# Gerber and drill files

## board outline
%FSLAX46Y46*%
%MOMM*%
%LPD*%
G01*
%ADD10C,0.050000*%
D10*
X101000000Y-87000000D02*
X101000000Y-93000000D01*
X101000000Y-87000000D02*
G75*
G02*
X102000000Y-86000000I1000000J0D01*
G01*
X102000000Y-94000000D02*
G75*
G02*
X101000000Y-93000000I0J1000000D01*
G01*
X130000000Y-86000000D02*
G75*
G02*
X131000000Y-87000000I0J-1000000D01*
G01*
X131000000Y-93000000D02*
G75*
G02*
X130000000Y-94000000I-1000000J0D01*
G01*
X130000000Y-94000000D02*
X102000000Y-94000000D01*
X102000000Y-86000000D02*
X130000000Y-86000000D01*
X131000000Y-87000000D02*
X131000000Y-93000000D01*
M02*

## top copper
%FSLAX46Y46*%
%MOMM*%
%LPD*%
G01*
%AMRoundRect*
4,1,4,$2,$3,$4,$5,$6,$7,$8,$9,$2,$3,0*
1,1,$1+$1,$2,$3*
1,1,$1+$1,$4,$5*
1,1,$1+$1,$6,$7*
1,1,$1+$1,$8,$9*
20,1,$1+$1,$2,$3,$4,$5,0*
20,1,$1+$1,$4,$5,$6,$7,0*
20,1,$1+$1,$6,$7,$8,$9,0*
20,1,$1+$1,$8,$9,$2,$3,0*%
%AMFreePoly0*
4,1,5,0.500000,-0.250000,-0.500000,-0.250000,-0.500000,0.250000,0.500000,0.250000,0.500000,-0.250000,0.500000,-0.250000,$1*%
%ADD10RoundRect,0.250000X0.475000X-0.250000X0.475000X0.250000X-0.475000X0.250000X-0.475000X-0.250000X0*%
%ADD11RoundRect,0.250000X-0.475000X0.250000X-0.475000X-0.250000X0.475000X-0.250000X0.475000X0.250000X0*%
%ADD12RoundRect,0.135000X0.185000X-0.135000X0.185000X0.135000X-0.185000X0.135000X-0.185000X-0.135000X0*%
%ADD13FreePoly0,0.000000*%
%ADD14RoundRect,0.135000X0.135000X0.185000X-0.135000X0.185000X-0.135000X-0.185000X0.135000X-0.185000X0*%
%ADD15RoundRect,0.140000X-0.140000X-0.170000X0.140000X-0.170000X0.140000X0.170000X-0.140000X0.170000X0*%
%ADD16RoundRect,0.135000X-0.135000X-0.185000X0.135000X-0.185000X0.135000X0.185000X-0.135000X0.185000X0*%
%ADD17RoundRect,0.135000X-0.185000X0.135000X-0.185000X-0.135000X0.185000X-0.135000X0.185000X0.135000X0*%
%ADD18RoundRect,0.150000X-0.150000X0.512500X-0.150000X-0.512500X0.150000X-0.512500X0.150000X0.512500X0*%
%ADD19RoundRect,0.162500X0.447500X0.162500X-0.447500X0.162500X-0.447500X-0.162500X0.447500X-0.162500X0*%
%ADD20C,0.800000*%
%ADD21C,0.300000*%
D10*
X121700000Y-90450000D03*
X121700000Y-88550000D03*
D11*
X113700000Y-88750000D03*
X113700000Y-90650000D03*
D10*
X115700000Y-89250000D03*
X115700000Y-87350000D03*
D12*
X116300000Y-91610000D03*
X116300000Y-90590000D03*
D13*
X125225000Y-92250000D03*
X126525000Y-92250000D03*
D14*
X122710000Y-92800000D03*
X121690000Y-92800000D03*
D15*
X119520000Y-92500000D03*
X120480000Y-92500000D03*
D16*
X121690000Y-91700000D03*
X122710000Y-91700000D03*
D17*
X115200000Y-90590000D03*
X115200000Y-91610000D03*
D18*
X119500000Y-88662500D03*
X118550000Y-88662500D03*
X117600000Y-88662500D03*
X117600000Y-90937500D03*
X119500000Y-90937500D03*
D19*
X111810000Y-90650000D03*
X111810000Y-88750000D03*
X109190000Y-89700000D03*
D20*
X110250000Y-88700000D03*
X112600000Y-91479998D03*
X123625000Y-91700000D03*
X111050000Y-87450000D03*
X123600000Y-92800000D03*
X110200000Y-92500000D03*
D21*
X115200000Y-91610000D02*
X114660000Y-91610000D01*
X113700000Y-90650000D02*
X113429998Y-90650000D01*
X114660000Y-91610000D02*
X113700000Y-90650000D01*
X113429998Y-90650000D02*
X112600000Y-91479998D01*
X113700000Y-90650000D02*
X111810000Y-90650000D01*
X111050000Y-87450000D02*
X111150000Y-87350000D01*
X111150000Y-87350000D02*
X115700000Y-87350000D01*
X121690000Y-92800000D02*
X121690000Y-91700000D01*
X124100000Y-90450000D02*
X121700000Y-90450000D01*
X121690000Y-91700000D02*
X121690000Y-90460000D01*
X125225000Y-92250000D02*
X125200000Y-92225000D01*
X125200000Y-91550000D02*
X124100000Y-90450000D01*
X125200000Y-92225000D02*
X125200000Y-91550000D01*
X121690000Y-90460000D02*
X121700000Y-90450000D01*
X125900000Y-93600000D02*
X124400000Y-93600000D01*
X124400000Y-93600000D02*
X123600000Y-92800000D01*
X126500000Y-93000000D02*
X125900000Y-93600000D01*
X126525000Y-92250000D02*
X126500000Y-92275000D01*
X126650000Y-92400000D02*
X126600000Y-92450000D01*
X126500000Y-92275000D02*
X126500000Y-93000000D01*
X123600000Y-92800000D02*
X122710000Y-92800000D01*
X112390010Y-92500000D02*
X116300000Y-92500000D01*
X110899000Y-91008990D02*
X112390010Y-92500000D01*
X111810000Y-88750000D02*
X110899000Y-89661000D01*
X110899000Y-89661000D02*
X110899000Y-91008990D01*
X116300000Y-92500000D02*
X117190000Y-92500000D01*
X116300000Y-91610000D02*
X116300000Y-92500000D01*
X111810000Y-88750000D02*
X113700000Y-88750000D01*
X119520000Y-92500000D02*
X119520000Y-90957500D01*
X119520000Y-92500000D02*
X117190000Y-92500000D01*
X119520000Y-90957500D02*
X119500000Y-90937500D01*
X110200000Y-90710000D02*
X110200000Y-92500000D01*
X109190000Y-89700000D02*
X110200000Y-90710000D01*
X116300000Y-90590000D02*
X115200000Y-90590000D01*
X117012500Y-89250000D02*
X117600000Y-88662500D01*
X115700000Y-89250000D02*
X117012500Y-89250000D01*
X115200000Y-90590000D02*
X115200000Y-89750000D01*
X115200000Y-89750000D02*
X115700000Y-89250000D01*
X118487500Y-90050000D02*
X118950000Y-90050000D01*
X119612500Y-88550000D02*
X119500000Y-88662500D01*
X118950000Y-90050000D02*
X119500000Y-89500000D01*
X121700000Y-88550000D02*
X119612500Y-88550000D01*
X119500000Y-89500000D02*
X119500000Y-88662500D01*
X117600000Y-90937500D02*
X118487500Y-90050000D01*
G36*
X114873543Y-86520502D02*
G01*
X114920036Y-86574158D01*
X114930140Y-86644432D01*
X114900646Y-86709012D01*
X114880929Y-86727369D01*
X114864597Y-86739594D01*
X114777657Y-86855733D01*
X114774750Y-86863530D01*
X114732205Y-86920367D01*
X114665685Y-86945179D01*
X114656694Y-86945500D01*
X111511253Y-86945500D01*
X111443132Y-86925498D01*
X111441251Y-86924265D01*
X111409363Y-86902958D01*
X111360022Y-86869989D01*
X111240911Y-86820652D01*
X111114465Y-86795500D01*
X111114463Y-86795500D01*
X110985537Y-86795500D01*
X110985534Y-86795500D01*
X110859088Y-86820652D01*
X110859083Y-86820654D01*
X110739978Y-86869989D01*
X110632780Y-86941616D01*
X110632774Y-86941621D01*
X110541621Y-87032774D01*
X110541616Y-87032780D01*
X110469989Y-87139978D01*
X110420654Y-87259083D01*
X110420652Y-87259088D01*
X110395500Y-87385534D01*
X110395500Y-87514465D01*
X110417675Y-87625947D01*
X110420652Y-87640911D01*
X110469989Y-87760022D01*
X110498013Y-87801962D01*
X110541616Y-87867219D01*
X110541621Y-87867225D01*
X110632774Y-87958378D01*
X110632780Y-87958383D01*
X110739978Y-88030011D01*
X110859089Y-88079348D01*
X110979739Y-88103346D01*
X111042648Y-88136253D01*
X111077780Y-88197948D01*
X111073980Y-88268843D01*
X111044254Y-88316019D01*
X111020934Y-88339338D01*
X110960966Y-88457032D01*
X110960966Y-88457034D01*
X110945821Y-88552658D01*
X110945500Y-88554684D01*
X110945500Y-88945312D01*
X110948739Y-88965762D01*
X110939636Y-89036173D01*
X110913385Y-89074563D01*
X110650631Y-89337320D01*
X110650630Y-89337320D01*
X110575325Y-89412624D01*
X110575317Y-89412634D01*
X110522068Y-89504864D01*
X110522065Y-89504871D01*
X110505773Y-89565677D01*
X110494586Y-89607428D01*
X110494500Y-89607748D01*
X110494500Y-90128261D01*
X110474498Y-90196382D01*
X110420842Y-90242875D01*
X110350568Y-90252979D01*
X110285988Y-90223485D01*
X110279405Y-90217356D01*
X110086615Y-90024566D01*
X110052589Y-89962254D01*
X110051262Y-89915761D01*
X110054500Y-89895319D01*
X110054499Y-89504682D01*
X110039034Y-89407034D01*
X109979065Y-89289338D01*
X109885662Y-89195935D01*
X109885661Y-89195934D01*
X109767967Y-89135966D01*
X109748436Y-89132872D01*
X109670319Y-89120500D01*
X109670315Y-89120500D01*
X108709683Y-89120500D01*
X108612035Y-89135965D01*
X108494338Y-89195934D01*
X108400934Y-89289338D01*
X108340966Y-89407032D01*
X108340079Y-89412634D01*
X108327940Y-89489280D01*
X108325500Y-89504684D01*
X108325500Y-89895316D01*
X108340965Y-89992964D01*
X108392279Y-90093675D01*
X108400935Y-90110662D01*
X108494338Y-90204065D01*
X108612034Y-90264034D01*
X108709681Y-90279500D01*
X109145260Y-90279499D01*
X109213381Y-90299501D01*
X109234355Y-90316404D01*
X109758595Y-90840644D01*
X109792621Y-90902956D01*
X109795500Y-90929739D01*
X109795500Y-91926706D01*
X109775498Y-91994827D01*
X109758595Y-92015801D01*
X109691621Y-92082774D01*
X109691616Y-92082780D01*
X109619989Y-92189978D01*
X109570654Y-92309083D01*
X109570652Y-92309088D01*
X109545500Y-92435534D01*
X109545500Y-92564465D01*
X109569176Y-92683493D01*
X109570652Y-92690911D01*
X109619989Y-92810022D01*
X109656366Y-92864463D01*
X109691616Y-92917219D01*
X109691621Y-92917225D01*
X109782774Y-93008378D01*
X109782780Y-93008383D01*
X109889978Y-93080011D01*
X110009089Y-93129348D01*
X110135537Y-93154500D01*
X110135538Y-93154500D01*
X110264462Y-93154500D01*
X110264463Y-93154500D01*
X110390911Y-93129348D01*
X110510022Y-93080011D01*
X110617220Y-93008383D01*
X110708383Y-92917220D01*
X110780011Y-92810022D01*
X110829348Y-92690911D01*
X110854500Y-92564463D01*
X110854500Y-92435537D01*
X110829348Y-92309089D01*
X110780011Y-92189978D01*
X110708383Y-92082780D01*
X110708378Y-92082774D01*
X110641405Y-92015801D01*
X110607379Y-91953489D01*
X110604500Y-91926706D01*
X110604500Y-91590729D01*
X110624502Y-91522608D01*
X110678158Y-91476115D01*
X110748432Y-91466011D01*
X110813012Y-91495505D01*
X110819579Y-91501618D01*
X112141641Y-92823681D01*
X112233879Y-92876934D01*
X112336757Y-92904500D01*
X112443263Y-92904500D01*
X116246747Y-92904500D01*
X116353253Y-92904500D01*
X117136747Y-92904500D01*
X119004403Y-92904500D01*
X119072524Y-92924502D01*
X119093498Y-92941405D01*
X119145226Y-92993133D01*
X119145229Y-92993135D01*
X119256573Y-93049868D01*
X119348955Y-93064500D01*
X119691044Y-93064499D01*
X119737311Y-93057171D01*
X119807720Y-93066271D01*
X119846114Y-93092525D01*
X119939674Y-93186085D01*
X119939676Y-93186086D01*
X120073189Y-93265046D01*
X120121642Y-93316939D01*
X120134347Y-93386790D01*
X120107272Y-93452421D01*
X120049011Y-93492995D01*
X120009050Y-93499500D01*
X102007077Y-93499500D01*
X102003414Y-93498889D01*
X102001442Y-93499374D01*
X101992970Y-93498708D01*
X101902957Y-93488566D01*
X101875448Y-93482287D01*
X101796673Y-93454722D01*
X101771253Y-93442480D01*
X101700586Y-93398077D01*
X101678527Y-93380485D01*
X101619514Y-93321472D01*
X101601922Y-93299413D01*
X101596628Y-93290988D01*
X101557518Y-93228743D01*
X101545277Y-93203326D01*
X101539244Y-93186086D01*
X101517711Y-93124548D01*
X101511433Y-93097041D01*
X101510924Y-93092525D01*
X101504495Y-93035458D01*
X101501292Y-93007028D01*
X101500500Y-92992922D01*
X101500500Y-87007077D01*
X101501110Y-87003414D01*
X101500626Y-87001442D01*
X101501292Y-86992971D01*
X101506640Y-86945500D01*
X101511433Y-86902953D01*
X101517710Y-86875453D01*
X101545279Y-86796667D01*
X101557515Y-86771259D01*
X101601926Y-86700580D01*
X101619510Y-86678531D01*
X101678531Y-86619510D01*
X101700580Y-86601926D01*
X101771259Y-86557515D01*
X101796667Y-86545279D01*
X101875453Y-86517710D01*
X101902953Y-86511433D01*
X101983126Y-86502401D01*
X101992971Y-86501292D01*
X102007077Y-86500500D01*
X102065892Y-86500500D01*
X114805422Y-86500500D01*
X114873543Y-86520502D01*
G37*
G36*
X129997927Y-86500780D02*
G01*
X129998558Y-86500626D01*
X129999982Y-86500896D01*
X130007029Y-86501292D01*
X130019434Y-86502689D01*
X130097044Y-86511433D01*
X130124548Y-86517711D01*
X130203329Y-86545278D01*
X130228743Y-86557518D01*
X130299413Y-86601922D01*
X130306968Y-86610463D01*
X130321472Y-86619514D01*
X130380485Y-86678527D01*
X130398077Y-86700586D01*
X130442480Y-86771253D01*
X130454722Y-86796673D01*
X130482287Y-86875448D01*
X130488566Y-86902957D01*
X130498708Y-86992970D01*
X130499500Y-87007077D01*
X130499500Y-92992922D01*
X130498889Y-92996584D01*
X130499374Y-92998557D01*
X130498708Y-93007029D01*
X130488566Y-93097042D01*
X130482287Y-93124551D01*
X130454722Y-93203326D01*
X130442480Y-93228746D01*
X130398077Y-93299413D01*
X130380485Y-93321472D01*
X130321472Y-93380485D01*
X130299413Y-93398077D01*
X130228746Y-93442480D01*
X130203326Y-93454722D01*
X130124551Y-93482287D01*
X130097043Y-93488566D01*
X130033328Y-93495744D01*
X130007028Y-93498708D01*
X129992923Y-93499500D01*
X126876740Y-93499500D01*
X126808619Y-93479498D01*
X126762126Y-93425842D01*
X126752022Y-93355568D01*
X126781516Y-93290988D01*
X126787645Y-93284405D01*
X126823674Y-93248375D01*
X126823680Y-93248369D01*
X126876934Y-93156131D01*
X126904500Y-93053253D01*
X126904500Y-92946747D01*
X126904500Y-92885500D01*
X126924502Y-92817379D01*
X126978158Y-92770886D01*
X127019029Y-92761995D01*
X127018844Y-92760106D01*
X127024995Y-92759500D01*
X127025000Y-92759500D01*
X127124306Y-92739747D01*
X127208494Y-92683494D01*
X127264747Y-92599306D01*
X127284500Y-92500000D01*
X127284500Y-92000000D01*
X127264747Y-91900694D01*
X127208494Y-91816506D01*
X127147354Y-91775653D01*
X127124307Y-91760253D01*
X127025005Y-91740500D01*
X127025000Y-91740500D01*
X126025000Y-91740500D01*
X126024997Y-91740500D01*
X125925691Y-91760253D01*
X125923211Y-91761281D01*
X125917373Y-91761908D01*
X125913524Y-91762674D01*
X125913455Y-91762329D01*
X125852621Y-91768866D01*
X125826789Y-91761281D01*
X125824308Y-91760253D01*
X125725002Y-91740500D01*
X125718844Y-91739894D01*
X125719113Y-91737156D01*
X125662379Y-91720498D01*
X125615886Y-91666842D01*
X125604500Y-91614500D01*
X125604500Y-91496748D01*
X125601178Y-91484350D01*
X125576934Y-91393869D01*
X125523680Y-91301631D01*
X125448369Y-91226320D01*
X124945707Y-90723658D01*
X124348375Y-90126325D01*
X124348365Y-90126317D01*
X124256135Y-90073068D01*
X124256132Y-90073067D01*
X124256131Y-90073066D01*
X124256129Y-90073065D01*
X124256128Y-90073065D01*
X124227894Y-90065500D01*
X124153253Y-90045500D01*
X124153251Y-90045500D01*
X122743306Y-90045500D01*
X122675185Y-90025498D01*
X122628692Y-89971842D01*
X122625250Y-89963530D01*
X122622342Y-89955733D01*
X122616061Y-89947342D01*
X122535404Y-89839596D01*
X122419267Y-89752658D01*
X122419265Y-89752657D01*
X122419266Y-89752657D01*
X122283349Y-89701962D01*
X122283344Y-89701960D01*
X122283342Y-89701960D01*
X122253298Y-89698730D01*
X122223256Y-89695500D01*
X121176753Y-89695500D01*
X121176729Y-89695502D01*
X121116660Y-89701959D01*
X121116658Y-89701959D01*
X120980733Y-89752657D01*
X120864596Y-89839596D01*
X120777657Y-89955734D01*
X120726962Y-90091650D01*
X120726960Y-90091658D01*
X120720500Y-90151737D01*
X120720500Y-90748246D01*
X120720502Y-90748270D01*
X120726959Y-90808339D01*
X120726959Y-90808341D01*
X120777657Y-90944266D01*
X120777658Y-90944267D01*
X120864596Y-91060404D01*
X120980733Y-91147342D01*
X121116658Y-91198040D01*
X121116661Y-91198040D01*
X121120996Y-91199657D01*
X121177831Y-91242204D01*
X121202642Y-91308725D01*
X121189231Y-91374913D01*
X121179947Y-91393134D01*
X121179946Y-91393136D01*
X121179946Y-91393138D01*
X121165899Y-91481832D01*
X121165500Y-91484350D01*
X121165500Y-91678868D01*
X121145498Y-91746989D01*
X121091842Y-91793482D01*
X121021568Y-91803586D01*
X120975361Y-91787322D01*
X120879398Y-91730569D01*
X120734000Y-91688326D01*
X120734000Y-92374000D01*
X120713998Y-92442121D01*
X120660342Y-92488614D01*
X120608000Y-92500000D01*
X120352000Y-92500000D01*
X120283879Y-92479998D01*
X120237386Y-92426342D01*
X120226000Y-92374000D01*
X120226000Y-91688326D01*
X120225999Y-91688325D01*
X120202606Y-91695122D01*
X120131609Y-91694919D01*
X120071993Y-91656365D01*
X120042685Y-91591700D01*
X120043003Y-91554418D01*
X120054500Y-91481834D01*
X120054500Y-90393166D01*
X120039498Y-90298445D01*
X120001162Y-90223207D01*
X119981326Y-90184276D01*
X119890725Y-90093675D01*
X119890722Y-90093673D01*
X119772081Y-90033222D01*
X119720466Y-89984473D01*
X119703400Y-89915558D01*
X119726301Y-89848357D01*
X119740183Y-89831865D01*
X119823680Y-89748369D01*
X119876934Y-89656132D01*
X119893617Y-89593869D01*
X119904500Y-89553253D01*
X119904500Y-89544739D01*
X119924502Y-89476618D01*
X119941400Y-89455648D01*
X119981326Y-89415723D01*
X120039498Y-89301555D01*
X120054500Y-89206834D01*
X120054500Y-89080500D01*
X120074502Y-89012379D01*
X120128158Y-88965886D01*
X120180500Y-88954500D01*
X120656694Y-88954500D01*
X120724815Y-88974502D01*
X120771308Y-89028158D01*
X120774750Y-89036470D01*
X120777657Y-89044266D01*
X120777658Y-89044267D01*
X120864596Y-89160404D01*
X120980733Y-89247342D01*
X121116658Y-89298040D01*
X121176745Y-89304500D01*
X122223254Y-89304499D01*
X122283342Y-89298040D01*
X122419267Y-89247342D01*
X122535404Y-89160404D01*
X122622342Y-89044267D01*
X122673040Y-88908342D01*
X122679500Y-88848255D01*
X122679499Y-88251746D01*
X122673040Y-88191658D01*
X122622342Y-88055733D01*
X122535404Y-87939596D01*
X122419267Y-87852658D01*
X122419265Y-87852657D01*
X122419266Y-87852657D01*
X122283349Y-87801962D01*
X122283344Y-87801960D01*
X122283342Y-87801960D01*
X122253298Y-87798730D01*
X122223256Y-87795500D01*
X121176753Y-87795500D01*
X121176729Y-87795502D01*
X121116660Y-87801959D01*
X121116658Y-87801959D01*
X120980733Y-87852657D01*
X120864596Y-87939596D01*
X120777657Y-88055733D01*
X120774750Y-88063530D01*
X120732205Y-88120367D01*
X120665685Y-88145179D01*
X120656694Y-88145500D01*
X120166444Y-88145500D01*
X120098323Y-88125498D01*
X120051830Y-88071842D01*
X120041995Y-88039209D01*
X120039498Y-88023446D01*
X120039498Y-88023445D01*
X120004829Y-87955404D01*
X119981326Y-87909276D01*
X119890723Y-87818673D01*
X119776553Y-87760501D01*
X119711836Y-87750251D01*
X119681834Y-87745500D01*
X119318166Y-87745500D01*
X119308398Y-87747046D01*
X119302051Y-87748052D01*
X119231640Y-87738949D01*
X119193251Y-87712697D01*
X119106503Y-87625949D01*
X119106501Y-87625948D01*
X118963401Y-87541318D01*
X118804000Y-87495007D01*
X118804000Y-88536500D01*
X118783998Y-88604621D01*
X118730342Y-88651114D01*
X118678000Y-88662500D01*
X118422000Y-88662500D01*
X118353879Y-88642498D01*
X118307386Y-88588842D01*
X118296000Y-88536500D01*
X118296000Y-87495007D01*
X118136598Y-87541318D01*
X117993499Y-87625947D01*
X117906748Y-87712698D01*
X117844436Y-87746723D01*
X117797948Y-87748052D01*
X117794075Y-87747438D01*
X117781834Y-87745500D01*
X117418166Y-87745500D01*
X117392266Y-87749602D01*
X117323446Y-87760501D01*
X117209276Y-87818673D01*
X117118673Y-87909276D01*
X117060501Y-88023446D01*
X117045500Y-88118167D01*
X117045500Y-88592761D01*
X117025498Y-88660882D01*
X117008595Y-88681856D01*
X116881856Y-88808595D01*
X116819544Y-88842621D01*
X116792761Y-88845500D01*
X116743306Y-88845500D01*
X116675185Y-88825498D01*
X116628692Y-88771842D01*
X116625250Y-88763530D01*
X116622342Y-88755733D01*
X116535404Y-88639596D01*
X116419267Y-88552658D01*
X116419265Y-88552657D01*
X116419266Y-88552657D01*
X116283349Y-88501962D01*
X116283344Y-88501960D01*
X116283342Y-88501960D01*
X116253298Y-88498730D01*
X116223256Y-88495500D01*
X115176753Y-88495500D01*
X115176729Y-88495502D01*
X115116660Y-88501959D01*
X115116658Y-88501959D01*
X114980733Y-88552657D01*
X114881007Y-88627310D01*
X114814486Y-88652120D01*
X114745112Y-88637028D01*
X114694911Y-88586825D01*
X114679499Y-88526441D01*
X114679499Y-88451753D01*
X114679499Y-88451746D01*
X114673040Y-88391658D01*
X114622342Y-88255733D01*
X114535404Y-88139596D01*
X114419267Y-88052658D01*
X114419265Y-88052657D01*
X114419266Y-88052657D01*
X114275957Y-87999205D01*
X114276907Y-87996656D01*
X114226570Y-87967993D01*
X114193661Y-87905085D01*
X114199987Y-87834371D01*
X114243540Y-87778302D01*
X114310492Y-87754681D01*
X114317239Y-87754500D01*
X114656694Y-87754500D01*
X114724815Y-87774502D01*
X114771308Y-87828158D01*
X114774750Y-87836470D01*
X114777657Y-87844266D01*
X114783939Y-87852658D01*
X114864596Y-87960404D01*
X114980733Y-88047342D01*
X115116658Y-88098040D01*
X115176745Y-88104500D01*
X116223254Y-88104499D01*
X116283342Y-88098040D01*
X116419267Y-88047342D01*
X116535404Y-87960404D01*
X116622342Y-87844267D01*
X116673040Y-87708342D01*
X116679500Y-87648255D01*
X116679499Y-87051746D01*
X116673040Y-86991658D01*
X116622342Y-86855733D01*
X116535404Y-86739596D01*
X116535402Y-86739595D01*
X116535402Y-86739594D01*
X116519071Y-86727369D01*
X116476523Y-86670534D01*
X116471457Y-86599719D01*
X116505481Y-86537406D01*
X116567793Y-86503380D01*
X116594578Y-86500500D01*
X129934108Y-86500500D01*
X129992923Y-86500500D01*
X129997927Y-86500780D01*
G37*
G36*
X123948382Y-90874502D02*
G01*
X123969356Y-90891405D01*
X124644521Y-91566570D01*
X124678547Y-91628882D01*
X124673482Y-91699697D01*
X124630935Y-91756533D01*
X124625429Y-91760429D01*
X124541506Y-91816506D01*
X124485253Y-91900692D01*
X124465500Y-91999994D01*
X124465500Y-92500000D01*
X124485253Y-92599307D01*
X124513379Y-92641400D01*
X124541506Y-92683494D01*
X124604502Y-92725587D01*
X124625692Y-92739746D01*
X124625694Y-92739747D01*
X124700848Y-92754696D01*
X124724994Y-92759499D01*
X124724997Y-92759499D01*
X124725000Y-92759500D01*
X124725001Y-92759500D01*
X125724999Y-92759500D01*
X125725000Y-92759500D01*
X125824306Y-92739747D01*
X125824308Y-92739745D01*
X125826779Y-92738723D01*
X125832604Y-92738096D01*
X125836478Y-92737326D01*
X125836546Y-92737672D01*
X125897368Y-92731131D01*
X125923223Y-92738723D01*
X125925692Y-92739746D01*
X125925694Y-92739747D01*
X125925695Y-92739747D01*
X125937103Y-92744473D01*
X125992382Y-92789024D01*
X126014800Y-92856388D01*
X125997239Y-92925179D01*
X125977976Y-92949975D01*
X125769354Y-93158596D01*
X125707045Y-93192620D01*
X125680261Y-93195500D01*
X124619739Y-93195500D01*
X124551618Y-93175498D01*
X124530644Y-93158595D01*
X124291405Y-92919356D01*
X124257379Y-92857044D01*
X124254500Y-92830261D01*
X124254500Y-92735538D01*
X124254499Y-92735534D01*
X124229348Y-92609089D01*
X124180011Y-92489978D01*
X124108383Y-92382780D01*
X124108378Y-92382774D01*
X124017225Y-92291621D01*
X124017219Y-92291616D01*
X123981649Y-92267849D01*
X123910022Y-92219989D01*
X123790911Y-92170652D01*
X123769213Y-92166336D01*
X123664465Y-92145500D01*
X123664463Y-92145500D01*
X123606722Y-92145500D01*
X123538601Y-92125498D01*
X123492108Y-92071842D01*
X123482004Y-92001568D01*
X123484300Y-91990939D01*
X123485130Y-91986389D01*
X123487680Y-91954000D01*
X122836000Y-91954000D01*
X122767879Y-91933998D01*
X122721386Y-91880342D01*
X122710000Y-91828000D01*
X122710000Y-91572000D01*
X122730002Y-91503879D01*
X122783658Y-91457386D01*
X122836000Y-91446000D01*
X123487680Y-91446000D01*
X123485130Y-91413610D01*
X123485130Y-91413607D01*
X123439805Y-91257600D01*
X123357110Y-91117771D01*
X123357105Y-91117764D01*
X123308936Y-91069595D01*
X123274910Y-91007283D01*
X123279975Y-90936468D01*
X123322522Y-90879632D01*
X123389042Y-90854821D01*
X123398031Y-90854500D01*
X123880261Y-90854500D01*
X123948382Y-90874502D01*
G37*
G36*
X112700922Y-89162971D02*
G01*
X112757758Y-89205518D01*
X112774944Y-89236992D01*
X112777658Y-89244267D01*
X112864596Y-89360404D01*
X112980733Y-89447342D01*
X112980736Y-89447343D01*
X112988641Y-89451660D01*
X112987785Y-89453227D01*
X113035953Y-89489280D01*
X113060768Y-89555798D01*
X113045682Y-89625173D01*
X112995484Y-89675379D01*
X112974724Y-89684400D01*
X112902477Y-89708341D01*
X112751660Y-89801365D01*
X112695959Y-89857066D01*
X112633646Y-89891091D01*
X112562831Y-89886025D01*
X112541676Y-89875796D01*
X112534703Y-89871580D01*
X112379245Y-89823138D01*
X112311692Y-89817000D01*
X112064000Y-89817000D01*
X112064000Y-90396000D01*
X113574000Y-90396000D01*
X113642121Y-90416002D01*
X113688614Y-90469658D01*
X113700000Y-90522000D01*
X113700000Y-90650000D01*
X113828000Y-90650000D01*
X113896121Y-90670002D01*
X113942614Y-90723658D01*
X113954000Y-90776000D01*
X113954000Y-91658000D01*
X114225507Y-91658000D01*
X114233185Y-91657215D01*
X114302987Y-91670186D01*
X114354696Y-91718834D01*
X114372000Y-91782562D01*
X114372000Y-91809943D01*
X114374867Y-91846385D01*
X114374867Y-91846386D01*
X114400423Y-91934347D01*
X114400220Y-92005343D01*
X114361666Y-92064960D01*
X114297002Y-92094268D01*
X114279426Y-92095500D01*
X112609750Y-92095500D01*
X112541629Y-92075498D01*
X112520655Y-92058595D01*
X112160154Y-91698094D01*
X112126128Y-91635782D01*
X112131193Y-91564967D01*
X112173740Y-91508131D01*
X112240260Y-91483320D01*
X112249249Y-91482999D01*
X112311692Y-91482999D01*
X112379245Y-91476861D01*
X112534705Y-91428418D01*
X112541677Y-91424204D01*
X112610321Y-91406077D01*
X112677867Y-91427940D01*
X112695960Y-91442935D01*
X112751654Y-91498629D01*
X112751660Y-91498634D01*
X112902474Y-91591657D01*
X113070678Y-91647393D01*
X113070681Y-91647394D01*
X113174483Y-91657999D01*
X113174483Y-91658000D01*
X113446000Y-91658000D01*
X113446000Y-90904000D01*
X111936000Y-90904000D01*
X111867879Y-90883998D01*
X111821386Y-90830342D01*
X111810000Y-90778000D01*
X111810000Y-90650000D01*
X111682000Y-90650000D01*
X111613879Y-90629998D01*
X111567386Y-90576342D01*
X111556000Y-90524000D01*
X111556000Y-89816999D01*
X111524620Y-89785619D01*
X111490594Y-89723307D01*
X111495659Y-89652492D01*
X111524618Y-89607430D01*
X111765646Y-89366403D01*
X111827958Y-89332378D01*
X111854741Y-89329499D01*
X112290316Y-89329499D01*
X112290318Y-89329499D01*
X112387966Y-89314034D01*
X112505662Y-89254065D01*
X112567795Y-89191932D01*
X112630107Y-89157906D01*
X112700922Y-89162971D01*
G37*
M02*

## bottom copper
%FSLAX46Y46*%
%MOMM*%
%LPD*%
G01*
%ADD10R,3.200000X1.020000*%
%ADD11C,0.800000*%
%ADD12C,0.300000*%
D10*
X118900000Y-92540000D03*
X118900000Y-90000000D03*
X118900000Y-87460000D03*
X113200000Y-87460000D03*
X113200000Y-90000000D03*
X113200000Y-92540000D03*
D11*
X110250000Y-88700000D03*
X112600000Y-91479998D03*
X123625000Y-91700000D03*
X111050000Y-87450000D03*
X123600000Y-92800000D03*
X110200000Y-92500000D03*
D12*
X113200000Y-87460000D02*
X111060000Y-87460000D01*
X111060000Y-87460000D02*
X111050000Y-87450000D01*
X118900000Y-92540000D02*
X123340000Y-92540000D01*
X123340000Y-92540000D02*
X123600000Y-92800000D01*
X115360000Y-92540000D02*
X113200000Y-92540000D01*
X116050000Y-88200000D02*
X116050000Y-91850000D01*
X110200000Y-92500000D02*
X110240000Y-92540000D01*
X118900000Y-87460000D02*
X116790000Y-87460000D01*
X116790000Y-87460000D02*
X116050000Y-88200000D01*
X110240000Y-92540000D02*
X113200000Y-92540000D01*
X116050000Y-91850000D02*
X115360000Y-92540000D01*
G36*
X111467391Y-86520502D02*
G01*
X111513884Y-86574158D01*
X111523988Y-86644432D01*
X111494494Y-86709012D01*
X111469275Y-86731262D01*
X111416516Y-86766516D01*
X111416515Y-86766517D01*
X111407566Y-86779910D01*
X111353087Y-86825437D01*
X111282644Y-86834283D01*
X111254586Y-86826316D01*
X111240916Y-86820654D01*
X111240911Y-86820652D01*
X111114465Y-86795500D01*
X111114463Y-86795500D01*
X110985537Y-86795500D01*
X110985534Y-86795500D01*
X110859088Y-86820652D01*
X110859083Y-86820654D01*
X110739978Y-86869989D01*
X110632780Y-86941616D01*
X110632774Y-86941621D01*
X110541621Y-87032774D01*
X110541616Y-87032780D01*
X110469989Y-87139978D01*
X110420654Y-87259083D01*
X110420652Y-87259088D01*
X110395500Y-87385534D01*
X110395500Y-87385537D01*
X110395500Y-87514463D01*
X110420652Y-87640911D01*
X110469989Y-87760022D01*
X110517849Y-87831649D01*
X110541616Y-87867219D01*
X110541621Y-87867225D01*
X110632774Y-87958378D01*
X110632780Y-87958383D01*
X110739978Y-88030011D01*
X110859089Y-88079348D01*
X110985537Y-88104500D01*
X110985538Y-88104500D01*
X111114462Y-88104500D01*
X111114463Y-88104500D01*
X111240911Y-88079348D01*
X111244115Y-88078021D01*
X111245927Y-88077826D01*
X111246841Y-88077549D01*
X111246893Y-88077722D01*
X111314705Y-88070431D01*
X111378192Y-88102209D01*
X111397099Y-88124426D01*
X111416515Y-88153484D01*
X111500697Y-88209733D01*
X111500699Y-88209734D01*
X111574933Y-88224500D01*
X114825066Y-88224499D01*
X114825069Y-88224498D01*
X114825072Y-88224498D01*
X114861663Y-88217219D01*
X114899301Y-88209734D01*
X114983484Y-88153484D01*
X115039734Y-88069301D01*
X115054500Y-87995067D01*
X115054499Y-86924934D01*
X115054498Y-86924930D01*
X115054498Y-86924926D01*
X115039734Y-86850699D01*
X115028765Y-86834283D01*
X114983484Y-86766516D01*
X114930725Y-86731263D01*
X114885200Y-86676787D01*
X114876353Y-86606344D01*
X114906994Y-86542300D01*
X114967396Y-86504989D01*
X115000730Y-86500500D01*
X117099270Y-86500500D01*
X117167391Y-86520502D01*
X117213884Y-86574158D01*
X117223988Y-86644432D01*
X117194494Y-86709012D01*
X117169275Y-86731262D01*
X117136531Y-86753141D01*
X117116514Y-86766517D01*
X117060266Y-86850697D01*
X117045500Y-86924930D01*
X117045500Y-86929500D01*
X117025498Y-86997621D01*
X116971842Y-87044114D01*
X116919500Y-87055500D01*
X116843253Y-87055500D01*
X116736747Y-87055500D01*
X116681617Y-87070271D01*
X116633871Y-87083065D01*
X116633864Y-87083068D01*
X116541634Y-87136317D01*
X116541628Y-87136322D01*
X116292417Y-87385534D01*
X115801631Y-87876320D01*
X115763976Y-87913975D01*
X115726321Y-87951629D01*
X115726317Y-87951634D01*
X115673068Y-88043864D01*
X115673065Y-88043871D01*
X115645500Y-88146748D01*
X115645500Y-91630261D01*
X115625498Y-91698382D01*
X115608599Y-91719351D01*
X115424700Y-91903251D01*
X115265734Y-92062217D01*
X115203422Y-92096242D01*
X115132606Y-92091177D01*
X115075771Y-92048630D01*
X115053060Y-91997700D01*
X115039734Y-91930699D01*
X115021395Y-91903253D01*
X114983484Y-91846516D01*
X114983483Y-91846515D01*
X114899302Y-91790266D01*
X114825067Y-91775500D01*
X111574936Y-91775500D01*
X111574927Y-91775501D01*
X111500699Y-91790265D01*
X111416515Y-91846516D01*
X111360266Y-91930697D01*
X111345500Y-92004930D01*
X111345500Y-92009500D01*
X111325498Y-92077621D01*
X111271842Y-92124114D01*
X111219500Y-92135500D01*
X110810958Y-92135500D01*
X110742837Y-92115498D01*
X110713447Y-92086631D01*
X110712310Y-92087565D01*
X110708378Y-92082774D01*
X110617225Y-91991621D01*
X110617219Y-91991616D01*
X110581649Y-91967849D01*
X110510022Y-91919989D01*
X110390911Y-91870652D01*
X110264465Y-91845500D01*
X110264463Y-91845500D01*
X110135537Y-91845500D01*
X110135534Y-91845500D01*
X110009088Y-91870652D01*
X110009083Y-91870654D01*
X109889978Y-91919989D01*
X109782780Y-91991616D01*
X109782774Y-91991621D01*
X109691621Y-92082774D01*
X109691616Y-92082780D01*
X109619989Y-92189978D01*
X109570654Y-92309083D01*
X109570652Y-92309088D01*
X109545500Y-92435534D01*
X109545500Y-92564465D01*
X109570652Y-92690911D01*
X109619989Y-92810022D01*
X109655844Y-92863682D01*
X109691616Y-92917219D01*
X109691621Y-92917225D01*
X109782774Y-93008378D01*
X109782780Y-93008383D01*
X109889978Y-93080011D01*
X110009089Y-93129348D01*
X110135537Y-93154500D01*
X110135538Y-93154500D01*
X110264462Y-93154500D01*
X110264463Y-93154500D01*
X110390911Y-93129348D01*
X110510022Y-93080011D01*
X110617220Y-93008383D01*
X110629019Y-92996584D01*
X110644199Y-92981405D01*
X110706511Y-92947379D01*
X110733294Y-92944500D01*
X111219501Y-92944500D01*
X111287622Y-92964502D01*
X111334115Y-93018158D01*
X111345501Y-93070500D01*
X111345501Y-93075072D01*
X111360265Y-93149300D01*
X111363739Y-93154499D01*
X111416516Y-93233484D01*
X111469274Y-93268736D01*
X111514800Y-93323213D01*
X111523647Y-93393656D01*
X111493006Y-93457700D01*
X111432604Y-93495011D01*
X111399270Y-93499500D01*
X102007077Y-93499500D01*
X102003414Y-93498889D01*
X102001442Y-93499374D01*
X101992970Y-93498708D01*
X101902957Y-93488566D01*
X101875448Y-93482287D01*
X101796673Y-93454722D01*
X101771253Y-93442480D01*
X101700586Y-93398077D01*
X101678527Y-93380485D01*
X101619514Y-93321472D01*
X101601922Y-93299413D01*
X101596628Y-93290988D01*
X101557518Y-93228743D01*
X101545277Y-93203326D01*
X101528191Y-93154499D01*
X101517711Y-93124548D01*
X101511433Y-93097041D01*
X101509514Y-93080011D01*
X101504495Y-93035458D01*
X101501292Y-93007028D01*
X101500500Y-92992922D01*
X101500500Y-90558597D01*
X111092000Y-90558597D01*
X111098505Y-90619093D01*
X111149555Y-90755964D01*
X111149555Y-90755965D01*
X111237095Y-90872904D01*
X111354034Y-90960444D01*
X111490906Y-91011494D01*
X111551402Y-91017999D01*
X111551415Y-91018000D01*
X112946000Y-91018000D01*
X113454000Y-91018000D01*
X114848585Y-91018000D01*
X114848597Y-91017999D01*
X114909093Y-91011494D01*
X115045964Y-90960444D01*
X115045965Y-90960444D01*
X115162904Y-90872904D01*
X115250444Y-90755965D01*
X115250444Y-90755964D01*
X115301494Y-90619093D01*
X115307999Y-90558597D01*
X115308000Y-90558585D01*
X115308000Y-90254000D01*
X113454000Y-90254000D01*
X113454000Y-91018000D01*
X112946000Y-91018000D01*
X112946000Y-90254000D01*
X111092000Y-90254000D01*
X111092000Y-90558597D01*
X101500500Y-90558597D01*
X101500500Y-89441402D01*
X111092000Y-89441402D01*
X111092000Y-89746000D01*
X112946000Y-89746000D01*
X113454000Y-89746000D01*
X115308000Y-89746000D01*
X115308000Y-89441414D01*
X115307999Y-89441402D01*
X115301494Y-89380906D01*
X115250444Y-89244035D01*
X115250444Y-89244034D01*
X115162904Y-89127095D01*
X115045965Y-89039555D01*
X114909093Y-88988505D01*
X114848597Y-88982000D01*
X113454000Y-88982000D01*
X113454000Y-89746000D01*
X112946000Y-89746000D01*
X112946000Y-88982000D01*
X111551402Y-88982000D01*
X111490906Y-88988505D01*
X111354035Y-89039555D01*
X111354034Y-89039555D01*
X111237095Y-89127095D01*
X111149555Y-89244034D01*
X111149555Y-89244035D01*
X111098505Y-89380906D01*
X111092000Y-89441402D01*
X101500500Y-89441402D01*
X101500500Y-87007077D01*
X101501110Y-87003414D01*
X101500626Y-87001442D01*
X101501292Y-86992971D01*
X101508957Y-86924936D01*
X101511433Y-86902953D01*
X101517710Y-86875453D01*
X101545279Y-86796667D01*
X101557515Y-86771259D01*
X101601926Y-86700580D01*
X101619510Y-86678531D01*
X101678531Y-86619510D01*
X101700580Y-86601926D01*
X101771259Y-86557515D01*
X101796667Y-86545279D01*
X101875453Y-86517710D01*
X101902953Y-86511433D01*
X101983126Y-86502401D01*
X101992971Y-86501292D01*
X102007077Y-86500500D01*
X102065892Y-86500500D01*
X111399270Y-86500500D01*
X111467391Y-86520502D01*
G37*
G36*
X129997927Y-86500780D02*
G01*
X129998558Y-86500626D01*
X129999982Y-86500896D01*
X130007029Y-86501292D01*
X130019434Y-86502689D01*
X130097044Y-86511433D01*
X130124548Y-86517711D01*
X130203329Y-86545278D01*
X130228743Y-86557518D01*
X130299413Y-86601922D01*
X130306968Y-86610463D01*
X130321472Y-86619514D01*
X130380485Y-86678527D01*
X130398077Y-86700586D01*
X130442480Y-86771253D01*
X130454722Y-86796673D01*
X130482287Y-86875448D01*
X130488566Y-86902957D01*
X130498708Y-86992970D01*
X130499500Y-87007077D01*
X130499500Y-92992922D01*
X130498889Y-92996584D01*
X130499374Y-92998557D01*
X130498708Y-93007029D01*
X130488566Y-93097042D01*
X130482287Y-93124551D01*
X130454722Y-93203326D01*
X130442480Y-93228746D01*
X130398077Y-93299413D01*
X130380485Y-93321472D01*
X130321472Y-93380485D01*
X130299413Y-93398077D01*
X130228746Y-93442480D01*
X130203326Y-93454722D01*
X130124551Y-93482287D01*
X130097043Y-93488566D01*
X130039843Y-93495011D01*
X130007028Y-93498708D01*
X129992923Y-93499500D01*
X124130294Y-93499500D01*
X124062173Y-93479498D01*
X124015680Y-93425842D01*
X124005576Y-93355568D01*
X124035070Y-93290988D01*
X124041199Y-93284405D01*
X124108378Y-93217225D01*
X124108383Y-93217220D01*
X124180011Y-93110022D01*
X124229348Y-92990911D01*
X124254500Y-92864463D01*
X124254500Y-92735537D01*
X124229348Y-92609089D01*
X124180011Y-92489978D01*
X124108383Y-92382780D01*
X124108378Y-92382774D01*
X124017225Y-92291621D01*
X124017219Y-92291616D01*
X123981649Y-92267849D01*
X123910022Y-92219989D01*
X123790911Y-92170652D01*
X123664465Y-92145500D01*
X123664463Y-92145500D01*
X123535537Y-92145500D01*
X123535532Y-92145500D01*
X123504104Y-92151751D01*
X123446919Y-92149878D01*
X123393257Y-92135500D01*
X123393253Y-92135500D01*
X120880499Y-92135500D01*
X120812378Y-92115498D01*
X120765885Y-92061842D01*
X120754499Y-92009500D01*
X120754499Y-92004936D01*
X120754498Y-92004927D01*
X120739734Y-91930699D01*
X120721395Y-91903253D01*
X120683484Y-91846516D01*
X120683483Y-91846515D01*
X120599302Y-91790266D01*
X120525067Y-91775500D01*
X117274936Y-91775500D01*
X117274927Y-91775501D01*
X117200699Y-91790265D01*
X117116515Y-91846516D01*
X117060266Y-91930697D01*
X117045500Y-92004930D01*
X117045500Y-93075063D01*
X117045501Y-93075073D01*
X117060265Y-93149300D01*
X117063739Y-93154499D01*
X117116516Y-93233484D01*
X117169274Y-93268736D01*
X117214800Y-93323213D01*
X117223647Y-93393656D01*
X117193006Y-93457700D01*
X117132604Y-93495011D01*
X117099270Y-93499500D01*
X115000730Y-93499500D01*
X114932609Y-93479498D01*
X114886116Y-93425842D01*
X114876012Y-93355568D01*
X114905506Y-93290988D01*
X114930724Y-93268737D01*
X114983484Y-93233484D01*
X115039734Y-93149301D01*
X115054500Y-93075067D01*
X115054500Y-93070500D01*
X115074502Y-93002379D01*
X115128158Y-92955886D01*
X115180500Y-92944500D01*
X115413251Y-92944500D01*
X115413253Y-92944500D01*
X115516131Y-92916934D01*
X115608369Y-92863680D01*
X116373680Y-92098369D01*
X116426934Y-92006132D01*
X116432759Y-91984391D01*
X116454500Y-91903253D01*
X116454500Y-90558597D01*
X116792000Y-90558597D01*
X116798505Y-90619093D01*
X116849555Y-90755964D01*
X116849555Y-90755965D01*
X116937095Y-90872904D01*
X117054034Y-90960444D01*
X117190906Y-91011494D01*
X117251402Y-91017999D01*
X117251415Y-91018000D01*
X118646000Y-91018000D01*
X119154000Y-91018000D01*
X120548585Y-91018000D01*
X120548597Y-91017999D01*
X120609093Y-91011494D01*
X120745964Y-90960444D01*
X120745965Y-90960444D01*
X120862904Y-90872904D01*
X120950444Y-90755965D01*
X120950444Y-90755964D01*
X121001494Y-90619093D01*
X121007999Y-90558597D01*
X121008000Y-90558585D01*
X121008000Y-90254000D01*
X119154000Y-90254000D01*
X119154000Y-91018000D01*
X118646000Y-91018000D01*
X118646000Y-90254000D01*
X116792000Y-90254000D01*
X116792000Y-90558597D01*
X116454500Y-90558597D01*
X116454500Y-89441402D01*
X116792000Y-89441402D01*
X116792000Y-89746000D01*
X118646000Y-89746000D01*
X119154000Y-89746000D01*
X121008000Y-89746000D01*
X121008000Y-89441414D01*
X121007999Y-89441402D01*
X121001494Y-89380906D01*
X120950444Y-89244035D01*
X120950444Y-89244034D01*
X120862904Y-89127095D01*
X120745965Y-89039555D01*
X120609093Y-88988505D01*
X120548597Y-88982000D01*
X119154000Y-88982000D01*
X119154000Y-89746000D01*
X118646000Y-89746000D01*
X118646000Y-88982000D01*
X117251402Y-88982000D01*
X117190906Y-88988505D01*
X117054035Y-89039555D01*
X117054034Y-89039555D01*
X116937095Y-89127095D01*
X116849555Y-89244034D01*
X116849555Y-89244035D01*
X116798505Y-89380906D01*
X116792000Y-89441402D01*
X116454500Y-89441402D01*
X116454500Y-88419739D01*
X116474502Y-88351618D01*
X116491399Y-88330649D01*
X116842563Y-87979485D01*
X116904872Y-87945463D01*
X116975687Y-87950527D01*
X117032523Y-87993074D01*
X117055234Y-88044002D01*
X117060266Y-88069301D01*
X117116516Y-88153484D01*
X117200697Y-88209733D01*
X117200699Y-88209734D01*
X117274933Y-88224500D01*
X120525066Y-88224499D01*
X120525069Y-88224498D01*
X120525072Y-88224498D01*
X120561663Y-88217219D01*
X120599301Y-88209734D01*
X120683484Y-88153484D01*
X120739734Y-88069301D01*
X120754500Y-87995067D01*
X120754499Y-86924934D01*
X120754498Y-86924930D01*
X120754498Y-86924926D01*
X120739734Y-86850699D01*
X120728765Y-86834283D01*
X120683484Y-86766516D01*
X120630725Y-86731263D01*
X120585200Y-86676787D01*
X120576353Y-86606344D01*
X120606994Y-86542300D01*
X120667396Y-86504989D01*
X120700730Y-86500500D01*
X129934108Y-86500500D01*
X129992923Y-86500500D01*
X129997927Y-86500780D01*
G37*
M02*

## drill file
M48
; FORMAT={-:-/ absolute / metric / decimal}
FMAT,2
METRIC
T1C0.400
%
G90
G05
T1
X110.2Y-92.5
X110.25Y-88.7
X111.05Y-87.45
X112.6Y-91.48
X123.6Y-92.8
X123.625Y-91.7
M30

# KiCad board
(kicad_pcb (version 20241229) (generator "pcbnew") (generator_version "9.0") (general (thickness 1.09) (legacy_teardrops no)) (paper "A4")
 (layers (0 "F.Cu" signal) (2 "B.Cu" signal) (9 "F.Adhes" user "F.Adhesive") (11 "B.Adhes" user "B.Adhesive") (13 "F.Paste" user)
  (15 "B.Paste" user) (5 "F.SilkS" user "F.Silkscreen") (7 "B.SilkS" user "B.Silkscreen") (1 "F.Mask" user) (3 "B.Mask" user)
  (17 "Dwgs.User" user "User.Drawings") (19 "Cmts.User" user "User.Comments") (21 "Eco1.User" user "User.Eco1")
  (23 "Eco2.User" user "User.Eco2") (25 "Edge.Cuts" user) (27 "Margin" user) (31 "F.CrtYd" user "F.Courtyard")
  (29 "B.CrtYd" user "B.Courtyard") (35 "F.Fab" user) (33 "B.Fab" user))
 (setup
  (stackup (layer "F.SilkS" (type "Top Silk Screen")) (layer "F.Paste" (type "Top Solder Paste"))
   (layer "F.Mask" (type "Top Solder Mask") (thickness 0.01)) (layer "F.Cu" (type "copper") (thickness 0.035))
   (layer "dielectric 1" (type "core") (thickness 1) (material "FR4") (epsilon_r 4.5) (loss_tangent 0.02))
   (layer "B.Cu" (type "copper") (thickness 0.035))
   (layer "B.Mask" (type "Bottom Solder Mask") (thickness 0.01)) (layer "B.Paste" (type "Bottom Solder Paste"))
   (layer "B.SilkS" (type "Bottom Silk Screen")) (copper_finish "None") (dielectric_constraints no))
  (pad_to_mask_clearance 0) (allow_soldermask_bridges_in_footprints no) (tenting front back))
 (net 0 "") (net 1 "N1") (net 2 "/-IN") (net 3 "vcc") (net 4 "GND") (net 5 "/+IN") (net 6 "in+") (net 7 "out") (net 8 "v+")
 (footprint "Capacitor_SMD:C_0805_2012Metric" (layer "F.Cu") (at 121.7 89.5 90)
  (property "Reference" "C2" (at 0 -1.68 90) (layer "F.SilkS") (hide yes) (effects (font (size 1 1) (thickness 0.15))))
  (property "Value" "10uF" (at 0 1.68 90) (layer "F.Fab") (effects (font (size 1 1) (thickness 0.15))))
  (pad "1" smd roundrect (at -0.95 0 90) (size 1 1.45) (layers "F.Cu" "F.Mask" "F.Paste") (roundrect_rratio 0.25) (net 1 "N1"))
  (pad "2" smd roundrect (at 0.95 0 90) (size 1 1.45) (layers "F.Cu" "F.Mask" "F.Paste") (roundrect_rratio 0.25) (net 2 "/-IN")))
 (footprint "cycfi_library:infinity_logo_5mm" (layer "F.Cu") (at 105.4 90)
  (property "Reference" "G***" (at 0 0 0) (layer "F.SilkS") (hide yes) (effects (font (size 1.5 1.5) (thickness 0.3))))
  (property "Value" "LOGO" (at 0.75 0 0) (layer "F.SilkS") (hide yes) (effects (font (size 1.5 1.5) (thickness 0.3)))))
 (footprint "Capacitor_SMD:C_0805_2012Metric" (layer "F.Cu") (at 113.7 89.7 -90)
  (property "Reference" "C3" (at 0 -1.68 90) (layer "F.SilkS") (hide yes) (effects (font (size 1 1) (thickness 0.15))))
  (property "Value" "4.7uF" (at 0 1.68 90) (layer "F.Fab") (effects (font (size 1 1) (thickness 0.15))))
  (pad "1" smd roundrect (at -0.95 0 270) (size 1 1.45) (layers "F.Cu" "F.Mask" "F.Paste") (roundrect_rratio 0.25) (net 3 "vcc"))
  (pad "2" smd roundrect (at 0.95 0 270) (size 1 1.45) (layers "F.Cu" "F.Mask" "F.Paste") (roundrect_rratio 0.25) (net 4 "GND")))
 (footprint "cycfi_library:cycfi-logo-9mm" (layer "F.Cu") (at 125.9 86.9)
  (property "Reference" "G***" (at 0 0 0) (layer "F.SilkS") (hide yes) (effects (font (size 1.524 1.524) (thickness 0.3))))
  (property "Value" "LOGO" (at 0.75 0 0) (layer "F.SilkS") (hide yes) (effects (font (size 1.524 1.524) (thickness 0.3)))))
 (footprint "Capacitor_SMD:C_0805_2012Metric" (layer "F.Cu") (at 115.7 88.3 90)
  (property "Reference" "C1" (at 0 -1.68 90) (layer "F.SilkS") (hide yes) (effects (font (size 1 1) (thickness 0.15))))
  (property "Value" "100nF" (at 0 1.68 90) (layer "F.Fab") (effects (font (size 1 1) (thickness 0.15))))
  (pad "1" smd roundrect (at -0.95 0 90) (size 1 1.45) (layers "F.Cu" "F.Mask" "F.Paste") (roundrect_rratio 0.25) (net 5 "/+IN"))
  (pad "2" smd roundrect (at 0.95 0 90) (size 1 1.45) (layers "F.Cu" "F.Mask" "F.Paste") (roundrect_rratio 0.25) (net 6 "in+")))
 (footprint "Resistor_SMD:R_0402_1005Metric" (layer "F.Cu") (at 116.3 91.1 90)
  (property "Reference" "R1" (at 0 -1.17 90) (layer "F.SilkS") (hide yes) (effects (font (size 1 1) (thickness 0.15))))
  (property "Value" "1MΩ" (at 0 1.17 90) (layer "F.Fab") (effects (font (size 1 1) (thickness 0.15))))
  (pad "1" smd roundrect (at -0.51 0 90) (size 0.54 0.64) (layers "F.Cu" "F.Mask" "F.Paste") (roundrect_rratio 0.25) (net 3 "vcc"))
  (pad "2" smd roundrect (at 0.51 0 90) (size 0.54 0.64) (layers "F.Cu" "F.Mask" "F.Paste") (roundrect_rratio 0.25) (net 5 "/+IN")))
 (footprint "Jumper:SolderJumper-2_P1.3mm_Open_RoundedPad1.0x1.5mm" (layer "F.Cu") (at 125.875 92.25)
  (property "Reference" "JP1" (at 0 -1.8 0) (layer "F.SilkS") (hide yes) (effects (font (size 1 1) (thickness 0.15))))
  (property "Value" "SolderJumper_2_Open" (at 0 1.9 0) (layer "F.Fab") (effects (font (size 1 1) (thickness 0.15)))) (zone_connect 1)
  (pad "1" smd custom (at -0.65 0) (size 1 0.5) (layers "F.Cu" "F.Mask") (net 1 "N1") (zone_connect 2) (thermal_bridge_angle 45)
   (options (clearance outline) (anchor rect)) (primitives))
  (pad "2" smd custom (at 0.65 0) (size 1 0.5) (layers "F.Cu" "F.Mask") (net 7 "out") (zone_connect 2) (thermal_bridge_angle 45)
   (options (clearance outline) (anchor rect)) (primitives)))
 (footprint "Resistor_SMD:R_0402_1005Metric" (layer "F.Cu") (at 122.2 92.8 180)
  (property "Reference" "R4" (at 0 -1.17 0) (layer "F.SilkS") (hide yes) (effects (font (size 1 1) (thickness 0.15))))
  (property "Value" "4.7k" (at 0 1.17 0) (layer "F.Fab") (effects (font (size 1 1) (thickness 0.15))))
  (pad "1" smd roundrect (at -0.51 0 180) (size 0.54 0.64) (layers "F.Cu" "F.Mask" "F.Paste") (roundrect_rratio 0.25) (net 7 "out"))
  (pad "2" smd roundrect (at 0.51 0 180) (size 0.54 0.64) (layers "F.Cu" "F.Mask" "F.Paste") (roundrect_rratio 0.25) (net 1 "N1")))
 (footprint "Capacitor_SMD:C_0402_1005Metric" (layer "F.Cu") (at 120 92.5)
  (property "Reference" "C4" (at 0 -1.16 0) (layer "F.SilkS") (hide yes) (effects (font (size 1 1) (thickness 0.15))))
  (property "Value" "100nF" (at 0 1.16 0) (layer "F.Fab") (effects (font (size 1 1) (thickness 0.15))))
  (pad "1" smd roundrect (at -0.48 0) (size 0.56 0.62) (layers "F.Cu" "F.Mask" "F.Paste") (roundrect_rratio 0.25) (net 3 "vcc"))
  (pad "2" smd roundrect (at 0.48 0) (size 0.56 0.62) (layers "F.Cu" "F.Mask" "F.Paste") (roundrect_rratio 0.25) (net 4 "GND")))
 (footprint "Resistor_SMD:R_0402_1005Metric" (layer "F.Cu") (at 122.2 91.7)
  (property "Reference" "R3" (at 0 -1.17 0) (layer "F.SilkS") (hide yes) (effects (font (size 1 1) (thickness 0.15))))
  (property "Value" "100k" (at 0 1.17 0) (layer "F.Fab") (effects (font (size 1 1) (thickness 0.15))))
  (pad "1" smd roundrect (at -0.51 0) (size 0.54 0.64) (layers "F.Cu" "F.Mask" "F.Paste") (roundrect_rratio 0.25) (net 1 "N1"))
  (pad "2" smd roundrect (at 0.51 0) (size 0.54 0.64) (layers "F.Cu" "F.Mask" "F.Paste") (roundrect_rratio 0.25) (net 4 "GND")))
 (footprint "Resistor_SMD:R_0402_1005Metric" (layer "F.Cu") (at 115.2 91.1 -90)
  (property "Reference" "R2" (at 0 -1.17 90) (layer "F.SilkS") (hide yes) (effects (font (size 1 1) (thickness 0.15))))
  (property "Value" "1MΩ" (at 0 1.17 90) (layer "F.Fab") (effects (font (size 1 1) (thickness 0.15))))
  (pad "1" smd roundrect (at -0.51 0 270) (size 0.54 0.64) (layers "F.Cu" "F.Mask" "F.Paste") (roundrect_rratio 0.25) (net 5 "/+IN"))
  (pad "2" smd roundrect (at 0.51 0 270) (size 0.54 0.64) (layers "F.Cu" "F.Mask" "F.Paste") (roundrect_rratio 0.25) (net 4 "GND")))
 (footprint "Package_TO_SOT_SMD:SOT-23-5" (layer "F.Cu") (at 118.55 89.8 -90)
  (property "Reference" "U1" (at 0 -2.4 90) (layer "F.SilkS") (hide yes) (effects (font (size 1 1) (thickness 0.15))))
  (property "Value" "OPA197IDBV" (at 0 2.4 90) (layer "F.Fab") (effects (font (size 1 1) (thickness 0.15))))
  (pad "1" smd roundrect (at -1.1375 -0.95 270) (size 1.325 0.6) (layers "F.Cu" "F.Mask" "F.Paste") (roundrect_rratio 0.25) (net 2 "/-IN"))
  (pad "2" smd roundrect (at -1.1375 0 270) (size 1.325 0.6) (layers "F.Cu" "F.Mask" "F.Paste") (roundrect_rratio 0.25) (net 4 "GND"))
  (pad "3" smd roundrect (at -1.1375 0.95 270) (size 1.325 0.6) (layers "F.Cu" "F.Mask" "F.Paste") (roundrect_rratio 0.25) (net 5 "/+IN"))
  (pad "4" smd roundrect (at 1.1375 0.95 270) (size 1.325 0.6) (layers "F.Cu" "F.Mask" "F.Paste") (roundrect_rratio 0.25) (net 2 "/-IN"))
  (pad "5" smd roundrect (at 1.1375 -0.95 270) (size 1.325 0.6) (layers "F.Cu" "F.Mask" "F.Paste") (roundrect_rratio 0.25) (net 3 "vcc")))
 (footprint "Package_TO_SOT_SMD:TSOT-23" (layer "F.Cu") (at 110.5 89.7 180)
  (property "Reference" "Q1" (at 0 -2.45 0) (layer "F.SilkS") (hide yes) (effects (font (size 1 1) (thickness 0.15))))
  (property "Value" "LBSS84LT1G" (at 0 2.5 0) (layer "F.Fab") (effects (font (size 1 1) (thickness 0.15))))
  (pad "1" smd roundrect (at -1.31 -0.95 180) (size 1.22 0.65) (layers "F.Cu" "F.Mask" "F.Paste") (roundrect_rratio 0.25) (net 4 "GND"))
  (pad "2" smd roundrect (at -1.31 0.95 180) (size 1.22 0.65) (layers "F.Cu" "F.Mask" "F.Paste") (roundrect_rratio 0.25) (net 3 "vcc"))
  (pad "3" smd roundrect (at 1.31 0 180) (size 1.22 0.65) (layers "F.Cu" "F.Mask" "F.Paste") (roundrect_rratio 0.25) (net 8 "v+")))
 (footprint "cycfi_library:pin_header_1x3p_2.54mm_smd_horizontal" (layer "B.Cu") (at 118.9 90)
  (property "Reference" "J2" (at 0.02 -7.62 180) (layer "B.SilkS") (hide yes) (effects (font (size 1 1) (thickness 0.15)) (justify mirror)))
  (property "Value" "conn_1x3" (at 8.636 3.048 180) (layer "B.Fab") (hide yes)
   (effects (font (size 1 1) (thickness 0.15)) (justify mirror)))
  (pad "1" smd rect (at 0 2.54) (size 3.2 1.02) (layers "B.Cu" "B.Mask" "B.Paste") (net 7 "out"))
  (pad "2" smd rect (at 0 0) (size 3.2 1.02) (layers "B.Cu" "B.Mask" "B.Paste") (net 4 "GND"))
  (pad "3" smd rect (at 0 -2.54) (size 3.2 1.02) (layers "B.Cu" "B.Mask" "B.Paste") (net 8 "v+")))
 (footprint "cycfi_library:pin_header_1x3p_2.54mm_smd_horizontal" (layer "B.Cu") (at 113.2 90 180)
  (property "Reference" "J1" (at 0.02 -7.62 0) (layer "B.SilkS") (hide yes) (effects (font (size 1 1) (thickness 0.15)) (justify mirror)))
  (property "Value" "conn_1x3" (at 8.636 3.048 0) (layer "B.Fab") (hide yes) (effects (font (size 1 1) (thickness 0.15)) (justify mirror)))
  (pad "1" smd rect (at 0 2.54 180) (size 3.2 1.02) (layers "B.Cu" "B.Mask" "B.Paste") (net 6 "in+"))
  (pad "2" smd rect (at 0 0 180) (size 3.2 1.02) (layers "B.Cu" "B.Mask" "B.Paste") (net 4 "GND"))
  (pad "3" smd rect (at 0 -2.54 180) (size 3.2 1.02) (layers "B.Cu" "B.Mask" "B.Paste") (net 8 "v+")))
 (gr_line (start 101 87) (end 101 93) (stroke (width 0.05) (type solid)) (layer "Edge.Cuts"))
 (gr_arc (start 101 87) (mid 101.292893 86.292893) (end 102 86) (stroke (width 0.05) (type solid)) (layer "Edge.Cuts"))
 (gr_arc (start 102 94) (mid 101.292893 93.707107) (end 101 93) (stroke (width 0.05) (type solid)) (layer "Edge.Cuts"))
 (gr_arc (start 130 86) (mid 130.707107 86.292893) (end 131 87) (stroke (width 0.05) (type solid)) (layer "Edge.Cuts"))
 (gr_arc (start 131 93) (mid 130.707107 93.707107) (end 130 94) (stroke (width 0.05) (type solid)) (layer "Edge.Cuts"))
 (gr_line (start 130 94) (end 102 94) (stroke (width 0.05) (type solid)) (layer "Edge.Cuts"))
 (gr_line (start 102 86) (end 130 86) (stroke (width 0.05) (type solid)) (layer "Edge.Cuts"))
 (gr_line (start 131 87) (end 131 93) (stroke (width 0.05) (type solid)) (layer "Edge.Cuts"))
 (segment (start 115.2 91.61) (end 114.66 91.61) (width 0.3) (layer "F.Cu") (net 4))
 (segment (start 113.7 90.65) (end 113.429998 90.65) (width 0.3) (layer "F.Cu") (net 4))
 (segment (start 114.66 91.61) (end 113.7 90.65) (width 0.3) (layer "F.Cu") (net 4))
 (segment (start 113.429998 90.65) (end 112.6 91.479998) (width 0.3) (layer "F.Cu") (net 4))
 (segment (start 113.7 90.65) (end 111.81 90.65) (width 0.3) (layer "F.Cu") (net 4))
 (via (at 110.25 88.7) (size 0.8) (drill 0.4) (layers "F.Cu" "B.Cu") (free yes) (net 4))
 (via (at 112.6 91.479998) (size 0.8) (drill 0.4) (layers "F.Cu" "B.Cu") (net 4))
 (via (at 123.625 91.7) (size 0.8) (drill 0.4) (layers "F.Cu" "B.Cu") (free yes) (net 4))
 (segment (start 111.05 87.45) (end 111.15 87.35) (width 0.3) (layer "F.Cu") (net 6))
 (segment (start 111.15 87.35) (end 115.7 87.35) (width 0.3) (layer "F.Cu") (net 6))
 (via (at 111.05 87.45) (size 0.8) (drill 0.4) (layers "F.Cu" "B.Cu") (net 6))
 (segment (start 113.2 87.46) (end 111.06 87.46) (width 0.3) (layer "B.Cu") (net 6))
 (segment (start 111.06 87.46) (end 111.05 87.45) (width 0.3) (layer "B.Cu") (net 6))
 (segment (start 121.69 92.8) (end 121.69 91.7) (width 0.3) (layer "F.Cu") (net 1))
 (segment (start 124.1 90.45) (end 121.7 90.45) (width 0.3) (layer "F.Cu") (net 1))
 (segment (start 121.69 91.7) (end 121.69 90.46) (width 0.3) (layer "F.Cu") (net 1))
 (segment (start 125.225 92.25) (end 125.2 92.225) (width 0.3) (layer "F.Cu") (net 1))
 (segment (start 125.2 91.55) (end 124.1 90.45) (width 0.3) (layer "F.Cu") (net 1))
 (segment (start 125.2 92.225) (end 125.2 91.55) (width 0.3) (layer "F.Cu") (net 1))
 (segment (start 121.69 90.46) (end 121.7 90.45) (width 0.3) (layer "F.Cu") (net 1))
 (segment (start 125.9 93.6) (end 124.4 93.6) (width 0.3) (layer "F.Cu") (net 7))
 (segment (start 124.4 93.6) (end 123.6 92.8) (width 0.3) (layer "F.Cu") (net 7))
 (segment (start 126.5 93) (end 125.9 93.6) (width 0.3) (layer "F.Cu") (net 7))
 (segment (start 126.525 92.25) (end 126.5 92.275) (width 0.3) (layer "F.Cu") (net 7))
 (segment (start 126.65 92.4) (end 126.6 92.45) (width 0.3) (layer "F.Cu") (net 7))
 (segment (start 126.5 92.275) (end 126.5 93) (width 0.3) (layer "F.Cu") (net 7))
 (segment (start 123.6 92.8) (end 122.71 92.8) (width 0.3) (layer "F.Cu") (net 7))
 (via (at 123.6 92.8) (size 0.8) (drill 0.4) (layers "F.Cu" "B.Cu") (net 7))
 (segment (start 118.9 92.54) (end 123.34 92.54) (width 0.3) (layer "B.Cu") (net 7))
 (segment (start 123.34 92.54) (end 123.6 92.8) (width 0.3) (layer "B.Cu") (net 7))
 (segment (start 112.39001 92.5) (end 116.3 92.5) (width 0.3) (layer "F.Cu") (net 3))
 (segment (start 110.899 91.00899) (end 112.39001 92.5) (width 0.3) (layer "F.Cu") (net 3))
 (segment (start 111.81 88.75) (end 110.899 89.661) (width 0.3) (layer "F.Cu") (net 3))
 (segment (start 110.899 89.661) (end 110.899 91.00899) (width 0.3) (layer "F.Cu") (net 3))
 (segment (start 116.3 92.5) (end 117.19 92.5) (width 0.3) (layer "F.Cu") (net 3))
 (segment (start 116.3 91.61) (end 116.3 92.5) (width 0.3) (layer "F.Cu") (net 3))
 (segment (start 111.81 88.75) (end 113.7 88.75) (width 0.3) (layer "F.Cu") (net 3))
 (segment (start 119.52 92.5) (end 119.52 90.9575) (width 0.3) (layer "F.Cu") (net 3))
 (segment (start 119.52 92.5) (end 117.19 92.5) (width 0.3) (layer "F.Cu") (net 3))
 (segment (start 119.52 90.9575) (end 119.5 90.9375) (width 0.3) (layer "F.Cu") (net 3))
 (segment (start 110.2 90.71) (end 110.2 92.5) (width 0.3) (layer "F.Cu") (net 8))
 (segment (start 109.19 89.7) (end 110.2 90.71) (width 0.3) (layer "F.Cu") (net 8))
 (via (at 110.2 92.5) (size 0.8) (drill 0.4) (layers "F.Cu" "B.Cu") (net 8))
 (segment (start 115.36 92.54) (end 113.2 92.54) (width 0.3) (layer "B.Cu") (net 8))
 (segment (start 116.05 88.2) (end 116.05 91.85) (width 0.3) (layer "B.Cu") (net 8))
 (segment (start 110.2 92.5) (end 110.24 92.54) (width 0.3) (layer "B.Cu") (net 8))
 (segment (start 118.9 87.46) (end 116.79 87.46) (width 0.3) (layer "B.Cu") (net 8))
 (segment (start 116.79 87.46) (end 116.05 88.2) (width 0.3) (layer "B.Cu") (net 8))
 (segment (start 110.24 92.54) (end 113.2 92.54) (width 0.3) (layer "B.Cu") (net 8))
 (segment (start 116.05 91.85) (end 115.36 92.54) (width 0.3) (layer "B.Cu") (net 8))
 (segment (start 116.3 90.59) (end 115.2 90.59) (width 0.3) (layer "F.Cu") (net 5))
 (segment (start 117.0125 89.25) (end 117.6 88.6625) (width 0.3) (layer "F.Cu") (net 5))
 (segment (start 115.7 89.25) (end 117.0125 89.25) (width 0.3) (layer "F.Cu") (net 5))
 (segment (start 115.2 90.59) (end 115.2 89.75) (width 0.3) (layer "F.Cu") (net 5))
 (segment (start 115.2 89.75) (end 115.7 89.25) (width 0.3) (layer "F.Cu") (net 5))
 (segment (start 118.4875 90.05) (end 118.95 90.05) (width 0.3) (layer "F.Cu") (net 2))
 (segment (start 119.6125 88.55) (end 119.5 88.6625) (width 0.3) (layer "F.Cu") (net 2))
 (segment (start 118.95 90.05) (end 119.5 89.5) (width 0.3) (layer "F.Cu") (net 2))
 (segment (start 121.7 88.55) (end 119.6125 88.55) (width 0.3) (layer "F.Cu") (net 2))
 (segment (start 119.5 89.5) (end 119.5 88.6625) (width 0.3) (layer "F.Cu") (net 2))
 (segment (start 117.6 90.9375) (end 118.4875 90.05) (width 0.3) (layer "F.Cu") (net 2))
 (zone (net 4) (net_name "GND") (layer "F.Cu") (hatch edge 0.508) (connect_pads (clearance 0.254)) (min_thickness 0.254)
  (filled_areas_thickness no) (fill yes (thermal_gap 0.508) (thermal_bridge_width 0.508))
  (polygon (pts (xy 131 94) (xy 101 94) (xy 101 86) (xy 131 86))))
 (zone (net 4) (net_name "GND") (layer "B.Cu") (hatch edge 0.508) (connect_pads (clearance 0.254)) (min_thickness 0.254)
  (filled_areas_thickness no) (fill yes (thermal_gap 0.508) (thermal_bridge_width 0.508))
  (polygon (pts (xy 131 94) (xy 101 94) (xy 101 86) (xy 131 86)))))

